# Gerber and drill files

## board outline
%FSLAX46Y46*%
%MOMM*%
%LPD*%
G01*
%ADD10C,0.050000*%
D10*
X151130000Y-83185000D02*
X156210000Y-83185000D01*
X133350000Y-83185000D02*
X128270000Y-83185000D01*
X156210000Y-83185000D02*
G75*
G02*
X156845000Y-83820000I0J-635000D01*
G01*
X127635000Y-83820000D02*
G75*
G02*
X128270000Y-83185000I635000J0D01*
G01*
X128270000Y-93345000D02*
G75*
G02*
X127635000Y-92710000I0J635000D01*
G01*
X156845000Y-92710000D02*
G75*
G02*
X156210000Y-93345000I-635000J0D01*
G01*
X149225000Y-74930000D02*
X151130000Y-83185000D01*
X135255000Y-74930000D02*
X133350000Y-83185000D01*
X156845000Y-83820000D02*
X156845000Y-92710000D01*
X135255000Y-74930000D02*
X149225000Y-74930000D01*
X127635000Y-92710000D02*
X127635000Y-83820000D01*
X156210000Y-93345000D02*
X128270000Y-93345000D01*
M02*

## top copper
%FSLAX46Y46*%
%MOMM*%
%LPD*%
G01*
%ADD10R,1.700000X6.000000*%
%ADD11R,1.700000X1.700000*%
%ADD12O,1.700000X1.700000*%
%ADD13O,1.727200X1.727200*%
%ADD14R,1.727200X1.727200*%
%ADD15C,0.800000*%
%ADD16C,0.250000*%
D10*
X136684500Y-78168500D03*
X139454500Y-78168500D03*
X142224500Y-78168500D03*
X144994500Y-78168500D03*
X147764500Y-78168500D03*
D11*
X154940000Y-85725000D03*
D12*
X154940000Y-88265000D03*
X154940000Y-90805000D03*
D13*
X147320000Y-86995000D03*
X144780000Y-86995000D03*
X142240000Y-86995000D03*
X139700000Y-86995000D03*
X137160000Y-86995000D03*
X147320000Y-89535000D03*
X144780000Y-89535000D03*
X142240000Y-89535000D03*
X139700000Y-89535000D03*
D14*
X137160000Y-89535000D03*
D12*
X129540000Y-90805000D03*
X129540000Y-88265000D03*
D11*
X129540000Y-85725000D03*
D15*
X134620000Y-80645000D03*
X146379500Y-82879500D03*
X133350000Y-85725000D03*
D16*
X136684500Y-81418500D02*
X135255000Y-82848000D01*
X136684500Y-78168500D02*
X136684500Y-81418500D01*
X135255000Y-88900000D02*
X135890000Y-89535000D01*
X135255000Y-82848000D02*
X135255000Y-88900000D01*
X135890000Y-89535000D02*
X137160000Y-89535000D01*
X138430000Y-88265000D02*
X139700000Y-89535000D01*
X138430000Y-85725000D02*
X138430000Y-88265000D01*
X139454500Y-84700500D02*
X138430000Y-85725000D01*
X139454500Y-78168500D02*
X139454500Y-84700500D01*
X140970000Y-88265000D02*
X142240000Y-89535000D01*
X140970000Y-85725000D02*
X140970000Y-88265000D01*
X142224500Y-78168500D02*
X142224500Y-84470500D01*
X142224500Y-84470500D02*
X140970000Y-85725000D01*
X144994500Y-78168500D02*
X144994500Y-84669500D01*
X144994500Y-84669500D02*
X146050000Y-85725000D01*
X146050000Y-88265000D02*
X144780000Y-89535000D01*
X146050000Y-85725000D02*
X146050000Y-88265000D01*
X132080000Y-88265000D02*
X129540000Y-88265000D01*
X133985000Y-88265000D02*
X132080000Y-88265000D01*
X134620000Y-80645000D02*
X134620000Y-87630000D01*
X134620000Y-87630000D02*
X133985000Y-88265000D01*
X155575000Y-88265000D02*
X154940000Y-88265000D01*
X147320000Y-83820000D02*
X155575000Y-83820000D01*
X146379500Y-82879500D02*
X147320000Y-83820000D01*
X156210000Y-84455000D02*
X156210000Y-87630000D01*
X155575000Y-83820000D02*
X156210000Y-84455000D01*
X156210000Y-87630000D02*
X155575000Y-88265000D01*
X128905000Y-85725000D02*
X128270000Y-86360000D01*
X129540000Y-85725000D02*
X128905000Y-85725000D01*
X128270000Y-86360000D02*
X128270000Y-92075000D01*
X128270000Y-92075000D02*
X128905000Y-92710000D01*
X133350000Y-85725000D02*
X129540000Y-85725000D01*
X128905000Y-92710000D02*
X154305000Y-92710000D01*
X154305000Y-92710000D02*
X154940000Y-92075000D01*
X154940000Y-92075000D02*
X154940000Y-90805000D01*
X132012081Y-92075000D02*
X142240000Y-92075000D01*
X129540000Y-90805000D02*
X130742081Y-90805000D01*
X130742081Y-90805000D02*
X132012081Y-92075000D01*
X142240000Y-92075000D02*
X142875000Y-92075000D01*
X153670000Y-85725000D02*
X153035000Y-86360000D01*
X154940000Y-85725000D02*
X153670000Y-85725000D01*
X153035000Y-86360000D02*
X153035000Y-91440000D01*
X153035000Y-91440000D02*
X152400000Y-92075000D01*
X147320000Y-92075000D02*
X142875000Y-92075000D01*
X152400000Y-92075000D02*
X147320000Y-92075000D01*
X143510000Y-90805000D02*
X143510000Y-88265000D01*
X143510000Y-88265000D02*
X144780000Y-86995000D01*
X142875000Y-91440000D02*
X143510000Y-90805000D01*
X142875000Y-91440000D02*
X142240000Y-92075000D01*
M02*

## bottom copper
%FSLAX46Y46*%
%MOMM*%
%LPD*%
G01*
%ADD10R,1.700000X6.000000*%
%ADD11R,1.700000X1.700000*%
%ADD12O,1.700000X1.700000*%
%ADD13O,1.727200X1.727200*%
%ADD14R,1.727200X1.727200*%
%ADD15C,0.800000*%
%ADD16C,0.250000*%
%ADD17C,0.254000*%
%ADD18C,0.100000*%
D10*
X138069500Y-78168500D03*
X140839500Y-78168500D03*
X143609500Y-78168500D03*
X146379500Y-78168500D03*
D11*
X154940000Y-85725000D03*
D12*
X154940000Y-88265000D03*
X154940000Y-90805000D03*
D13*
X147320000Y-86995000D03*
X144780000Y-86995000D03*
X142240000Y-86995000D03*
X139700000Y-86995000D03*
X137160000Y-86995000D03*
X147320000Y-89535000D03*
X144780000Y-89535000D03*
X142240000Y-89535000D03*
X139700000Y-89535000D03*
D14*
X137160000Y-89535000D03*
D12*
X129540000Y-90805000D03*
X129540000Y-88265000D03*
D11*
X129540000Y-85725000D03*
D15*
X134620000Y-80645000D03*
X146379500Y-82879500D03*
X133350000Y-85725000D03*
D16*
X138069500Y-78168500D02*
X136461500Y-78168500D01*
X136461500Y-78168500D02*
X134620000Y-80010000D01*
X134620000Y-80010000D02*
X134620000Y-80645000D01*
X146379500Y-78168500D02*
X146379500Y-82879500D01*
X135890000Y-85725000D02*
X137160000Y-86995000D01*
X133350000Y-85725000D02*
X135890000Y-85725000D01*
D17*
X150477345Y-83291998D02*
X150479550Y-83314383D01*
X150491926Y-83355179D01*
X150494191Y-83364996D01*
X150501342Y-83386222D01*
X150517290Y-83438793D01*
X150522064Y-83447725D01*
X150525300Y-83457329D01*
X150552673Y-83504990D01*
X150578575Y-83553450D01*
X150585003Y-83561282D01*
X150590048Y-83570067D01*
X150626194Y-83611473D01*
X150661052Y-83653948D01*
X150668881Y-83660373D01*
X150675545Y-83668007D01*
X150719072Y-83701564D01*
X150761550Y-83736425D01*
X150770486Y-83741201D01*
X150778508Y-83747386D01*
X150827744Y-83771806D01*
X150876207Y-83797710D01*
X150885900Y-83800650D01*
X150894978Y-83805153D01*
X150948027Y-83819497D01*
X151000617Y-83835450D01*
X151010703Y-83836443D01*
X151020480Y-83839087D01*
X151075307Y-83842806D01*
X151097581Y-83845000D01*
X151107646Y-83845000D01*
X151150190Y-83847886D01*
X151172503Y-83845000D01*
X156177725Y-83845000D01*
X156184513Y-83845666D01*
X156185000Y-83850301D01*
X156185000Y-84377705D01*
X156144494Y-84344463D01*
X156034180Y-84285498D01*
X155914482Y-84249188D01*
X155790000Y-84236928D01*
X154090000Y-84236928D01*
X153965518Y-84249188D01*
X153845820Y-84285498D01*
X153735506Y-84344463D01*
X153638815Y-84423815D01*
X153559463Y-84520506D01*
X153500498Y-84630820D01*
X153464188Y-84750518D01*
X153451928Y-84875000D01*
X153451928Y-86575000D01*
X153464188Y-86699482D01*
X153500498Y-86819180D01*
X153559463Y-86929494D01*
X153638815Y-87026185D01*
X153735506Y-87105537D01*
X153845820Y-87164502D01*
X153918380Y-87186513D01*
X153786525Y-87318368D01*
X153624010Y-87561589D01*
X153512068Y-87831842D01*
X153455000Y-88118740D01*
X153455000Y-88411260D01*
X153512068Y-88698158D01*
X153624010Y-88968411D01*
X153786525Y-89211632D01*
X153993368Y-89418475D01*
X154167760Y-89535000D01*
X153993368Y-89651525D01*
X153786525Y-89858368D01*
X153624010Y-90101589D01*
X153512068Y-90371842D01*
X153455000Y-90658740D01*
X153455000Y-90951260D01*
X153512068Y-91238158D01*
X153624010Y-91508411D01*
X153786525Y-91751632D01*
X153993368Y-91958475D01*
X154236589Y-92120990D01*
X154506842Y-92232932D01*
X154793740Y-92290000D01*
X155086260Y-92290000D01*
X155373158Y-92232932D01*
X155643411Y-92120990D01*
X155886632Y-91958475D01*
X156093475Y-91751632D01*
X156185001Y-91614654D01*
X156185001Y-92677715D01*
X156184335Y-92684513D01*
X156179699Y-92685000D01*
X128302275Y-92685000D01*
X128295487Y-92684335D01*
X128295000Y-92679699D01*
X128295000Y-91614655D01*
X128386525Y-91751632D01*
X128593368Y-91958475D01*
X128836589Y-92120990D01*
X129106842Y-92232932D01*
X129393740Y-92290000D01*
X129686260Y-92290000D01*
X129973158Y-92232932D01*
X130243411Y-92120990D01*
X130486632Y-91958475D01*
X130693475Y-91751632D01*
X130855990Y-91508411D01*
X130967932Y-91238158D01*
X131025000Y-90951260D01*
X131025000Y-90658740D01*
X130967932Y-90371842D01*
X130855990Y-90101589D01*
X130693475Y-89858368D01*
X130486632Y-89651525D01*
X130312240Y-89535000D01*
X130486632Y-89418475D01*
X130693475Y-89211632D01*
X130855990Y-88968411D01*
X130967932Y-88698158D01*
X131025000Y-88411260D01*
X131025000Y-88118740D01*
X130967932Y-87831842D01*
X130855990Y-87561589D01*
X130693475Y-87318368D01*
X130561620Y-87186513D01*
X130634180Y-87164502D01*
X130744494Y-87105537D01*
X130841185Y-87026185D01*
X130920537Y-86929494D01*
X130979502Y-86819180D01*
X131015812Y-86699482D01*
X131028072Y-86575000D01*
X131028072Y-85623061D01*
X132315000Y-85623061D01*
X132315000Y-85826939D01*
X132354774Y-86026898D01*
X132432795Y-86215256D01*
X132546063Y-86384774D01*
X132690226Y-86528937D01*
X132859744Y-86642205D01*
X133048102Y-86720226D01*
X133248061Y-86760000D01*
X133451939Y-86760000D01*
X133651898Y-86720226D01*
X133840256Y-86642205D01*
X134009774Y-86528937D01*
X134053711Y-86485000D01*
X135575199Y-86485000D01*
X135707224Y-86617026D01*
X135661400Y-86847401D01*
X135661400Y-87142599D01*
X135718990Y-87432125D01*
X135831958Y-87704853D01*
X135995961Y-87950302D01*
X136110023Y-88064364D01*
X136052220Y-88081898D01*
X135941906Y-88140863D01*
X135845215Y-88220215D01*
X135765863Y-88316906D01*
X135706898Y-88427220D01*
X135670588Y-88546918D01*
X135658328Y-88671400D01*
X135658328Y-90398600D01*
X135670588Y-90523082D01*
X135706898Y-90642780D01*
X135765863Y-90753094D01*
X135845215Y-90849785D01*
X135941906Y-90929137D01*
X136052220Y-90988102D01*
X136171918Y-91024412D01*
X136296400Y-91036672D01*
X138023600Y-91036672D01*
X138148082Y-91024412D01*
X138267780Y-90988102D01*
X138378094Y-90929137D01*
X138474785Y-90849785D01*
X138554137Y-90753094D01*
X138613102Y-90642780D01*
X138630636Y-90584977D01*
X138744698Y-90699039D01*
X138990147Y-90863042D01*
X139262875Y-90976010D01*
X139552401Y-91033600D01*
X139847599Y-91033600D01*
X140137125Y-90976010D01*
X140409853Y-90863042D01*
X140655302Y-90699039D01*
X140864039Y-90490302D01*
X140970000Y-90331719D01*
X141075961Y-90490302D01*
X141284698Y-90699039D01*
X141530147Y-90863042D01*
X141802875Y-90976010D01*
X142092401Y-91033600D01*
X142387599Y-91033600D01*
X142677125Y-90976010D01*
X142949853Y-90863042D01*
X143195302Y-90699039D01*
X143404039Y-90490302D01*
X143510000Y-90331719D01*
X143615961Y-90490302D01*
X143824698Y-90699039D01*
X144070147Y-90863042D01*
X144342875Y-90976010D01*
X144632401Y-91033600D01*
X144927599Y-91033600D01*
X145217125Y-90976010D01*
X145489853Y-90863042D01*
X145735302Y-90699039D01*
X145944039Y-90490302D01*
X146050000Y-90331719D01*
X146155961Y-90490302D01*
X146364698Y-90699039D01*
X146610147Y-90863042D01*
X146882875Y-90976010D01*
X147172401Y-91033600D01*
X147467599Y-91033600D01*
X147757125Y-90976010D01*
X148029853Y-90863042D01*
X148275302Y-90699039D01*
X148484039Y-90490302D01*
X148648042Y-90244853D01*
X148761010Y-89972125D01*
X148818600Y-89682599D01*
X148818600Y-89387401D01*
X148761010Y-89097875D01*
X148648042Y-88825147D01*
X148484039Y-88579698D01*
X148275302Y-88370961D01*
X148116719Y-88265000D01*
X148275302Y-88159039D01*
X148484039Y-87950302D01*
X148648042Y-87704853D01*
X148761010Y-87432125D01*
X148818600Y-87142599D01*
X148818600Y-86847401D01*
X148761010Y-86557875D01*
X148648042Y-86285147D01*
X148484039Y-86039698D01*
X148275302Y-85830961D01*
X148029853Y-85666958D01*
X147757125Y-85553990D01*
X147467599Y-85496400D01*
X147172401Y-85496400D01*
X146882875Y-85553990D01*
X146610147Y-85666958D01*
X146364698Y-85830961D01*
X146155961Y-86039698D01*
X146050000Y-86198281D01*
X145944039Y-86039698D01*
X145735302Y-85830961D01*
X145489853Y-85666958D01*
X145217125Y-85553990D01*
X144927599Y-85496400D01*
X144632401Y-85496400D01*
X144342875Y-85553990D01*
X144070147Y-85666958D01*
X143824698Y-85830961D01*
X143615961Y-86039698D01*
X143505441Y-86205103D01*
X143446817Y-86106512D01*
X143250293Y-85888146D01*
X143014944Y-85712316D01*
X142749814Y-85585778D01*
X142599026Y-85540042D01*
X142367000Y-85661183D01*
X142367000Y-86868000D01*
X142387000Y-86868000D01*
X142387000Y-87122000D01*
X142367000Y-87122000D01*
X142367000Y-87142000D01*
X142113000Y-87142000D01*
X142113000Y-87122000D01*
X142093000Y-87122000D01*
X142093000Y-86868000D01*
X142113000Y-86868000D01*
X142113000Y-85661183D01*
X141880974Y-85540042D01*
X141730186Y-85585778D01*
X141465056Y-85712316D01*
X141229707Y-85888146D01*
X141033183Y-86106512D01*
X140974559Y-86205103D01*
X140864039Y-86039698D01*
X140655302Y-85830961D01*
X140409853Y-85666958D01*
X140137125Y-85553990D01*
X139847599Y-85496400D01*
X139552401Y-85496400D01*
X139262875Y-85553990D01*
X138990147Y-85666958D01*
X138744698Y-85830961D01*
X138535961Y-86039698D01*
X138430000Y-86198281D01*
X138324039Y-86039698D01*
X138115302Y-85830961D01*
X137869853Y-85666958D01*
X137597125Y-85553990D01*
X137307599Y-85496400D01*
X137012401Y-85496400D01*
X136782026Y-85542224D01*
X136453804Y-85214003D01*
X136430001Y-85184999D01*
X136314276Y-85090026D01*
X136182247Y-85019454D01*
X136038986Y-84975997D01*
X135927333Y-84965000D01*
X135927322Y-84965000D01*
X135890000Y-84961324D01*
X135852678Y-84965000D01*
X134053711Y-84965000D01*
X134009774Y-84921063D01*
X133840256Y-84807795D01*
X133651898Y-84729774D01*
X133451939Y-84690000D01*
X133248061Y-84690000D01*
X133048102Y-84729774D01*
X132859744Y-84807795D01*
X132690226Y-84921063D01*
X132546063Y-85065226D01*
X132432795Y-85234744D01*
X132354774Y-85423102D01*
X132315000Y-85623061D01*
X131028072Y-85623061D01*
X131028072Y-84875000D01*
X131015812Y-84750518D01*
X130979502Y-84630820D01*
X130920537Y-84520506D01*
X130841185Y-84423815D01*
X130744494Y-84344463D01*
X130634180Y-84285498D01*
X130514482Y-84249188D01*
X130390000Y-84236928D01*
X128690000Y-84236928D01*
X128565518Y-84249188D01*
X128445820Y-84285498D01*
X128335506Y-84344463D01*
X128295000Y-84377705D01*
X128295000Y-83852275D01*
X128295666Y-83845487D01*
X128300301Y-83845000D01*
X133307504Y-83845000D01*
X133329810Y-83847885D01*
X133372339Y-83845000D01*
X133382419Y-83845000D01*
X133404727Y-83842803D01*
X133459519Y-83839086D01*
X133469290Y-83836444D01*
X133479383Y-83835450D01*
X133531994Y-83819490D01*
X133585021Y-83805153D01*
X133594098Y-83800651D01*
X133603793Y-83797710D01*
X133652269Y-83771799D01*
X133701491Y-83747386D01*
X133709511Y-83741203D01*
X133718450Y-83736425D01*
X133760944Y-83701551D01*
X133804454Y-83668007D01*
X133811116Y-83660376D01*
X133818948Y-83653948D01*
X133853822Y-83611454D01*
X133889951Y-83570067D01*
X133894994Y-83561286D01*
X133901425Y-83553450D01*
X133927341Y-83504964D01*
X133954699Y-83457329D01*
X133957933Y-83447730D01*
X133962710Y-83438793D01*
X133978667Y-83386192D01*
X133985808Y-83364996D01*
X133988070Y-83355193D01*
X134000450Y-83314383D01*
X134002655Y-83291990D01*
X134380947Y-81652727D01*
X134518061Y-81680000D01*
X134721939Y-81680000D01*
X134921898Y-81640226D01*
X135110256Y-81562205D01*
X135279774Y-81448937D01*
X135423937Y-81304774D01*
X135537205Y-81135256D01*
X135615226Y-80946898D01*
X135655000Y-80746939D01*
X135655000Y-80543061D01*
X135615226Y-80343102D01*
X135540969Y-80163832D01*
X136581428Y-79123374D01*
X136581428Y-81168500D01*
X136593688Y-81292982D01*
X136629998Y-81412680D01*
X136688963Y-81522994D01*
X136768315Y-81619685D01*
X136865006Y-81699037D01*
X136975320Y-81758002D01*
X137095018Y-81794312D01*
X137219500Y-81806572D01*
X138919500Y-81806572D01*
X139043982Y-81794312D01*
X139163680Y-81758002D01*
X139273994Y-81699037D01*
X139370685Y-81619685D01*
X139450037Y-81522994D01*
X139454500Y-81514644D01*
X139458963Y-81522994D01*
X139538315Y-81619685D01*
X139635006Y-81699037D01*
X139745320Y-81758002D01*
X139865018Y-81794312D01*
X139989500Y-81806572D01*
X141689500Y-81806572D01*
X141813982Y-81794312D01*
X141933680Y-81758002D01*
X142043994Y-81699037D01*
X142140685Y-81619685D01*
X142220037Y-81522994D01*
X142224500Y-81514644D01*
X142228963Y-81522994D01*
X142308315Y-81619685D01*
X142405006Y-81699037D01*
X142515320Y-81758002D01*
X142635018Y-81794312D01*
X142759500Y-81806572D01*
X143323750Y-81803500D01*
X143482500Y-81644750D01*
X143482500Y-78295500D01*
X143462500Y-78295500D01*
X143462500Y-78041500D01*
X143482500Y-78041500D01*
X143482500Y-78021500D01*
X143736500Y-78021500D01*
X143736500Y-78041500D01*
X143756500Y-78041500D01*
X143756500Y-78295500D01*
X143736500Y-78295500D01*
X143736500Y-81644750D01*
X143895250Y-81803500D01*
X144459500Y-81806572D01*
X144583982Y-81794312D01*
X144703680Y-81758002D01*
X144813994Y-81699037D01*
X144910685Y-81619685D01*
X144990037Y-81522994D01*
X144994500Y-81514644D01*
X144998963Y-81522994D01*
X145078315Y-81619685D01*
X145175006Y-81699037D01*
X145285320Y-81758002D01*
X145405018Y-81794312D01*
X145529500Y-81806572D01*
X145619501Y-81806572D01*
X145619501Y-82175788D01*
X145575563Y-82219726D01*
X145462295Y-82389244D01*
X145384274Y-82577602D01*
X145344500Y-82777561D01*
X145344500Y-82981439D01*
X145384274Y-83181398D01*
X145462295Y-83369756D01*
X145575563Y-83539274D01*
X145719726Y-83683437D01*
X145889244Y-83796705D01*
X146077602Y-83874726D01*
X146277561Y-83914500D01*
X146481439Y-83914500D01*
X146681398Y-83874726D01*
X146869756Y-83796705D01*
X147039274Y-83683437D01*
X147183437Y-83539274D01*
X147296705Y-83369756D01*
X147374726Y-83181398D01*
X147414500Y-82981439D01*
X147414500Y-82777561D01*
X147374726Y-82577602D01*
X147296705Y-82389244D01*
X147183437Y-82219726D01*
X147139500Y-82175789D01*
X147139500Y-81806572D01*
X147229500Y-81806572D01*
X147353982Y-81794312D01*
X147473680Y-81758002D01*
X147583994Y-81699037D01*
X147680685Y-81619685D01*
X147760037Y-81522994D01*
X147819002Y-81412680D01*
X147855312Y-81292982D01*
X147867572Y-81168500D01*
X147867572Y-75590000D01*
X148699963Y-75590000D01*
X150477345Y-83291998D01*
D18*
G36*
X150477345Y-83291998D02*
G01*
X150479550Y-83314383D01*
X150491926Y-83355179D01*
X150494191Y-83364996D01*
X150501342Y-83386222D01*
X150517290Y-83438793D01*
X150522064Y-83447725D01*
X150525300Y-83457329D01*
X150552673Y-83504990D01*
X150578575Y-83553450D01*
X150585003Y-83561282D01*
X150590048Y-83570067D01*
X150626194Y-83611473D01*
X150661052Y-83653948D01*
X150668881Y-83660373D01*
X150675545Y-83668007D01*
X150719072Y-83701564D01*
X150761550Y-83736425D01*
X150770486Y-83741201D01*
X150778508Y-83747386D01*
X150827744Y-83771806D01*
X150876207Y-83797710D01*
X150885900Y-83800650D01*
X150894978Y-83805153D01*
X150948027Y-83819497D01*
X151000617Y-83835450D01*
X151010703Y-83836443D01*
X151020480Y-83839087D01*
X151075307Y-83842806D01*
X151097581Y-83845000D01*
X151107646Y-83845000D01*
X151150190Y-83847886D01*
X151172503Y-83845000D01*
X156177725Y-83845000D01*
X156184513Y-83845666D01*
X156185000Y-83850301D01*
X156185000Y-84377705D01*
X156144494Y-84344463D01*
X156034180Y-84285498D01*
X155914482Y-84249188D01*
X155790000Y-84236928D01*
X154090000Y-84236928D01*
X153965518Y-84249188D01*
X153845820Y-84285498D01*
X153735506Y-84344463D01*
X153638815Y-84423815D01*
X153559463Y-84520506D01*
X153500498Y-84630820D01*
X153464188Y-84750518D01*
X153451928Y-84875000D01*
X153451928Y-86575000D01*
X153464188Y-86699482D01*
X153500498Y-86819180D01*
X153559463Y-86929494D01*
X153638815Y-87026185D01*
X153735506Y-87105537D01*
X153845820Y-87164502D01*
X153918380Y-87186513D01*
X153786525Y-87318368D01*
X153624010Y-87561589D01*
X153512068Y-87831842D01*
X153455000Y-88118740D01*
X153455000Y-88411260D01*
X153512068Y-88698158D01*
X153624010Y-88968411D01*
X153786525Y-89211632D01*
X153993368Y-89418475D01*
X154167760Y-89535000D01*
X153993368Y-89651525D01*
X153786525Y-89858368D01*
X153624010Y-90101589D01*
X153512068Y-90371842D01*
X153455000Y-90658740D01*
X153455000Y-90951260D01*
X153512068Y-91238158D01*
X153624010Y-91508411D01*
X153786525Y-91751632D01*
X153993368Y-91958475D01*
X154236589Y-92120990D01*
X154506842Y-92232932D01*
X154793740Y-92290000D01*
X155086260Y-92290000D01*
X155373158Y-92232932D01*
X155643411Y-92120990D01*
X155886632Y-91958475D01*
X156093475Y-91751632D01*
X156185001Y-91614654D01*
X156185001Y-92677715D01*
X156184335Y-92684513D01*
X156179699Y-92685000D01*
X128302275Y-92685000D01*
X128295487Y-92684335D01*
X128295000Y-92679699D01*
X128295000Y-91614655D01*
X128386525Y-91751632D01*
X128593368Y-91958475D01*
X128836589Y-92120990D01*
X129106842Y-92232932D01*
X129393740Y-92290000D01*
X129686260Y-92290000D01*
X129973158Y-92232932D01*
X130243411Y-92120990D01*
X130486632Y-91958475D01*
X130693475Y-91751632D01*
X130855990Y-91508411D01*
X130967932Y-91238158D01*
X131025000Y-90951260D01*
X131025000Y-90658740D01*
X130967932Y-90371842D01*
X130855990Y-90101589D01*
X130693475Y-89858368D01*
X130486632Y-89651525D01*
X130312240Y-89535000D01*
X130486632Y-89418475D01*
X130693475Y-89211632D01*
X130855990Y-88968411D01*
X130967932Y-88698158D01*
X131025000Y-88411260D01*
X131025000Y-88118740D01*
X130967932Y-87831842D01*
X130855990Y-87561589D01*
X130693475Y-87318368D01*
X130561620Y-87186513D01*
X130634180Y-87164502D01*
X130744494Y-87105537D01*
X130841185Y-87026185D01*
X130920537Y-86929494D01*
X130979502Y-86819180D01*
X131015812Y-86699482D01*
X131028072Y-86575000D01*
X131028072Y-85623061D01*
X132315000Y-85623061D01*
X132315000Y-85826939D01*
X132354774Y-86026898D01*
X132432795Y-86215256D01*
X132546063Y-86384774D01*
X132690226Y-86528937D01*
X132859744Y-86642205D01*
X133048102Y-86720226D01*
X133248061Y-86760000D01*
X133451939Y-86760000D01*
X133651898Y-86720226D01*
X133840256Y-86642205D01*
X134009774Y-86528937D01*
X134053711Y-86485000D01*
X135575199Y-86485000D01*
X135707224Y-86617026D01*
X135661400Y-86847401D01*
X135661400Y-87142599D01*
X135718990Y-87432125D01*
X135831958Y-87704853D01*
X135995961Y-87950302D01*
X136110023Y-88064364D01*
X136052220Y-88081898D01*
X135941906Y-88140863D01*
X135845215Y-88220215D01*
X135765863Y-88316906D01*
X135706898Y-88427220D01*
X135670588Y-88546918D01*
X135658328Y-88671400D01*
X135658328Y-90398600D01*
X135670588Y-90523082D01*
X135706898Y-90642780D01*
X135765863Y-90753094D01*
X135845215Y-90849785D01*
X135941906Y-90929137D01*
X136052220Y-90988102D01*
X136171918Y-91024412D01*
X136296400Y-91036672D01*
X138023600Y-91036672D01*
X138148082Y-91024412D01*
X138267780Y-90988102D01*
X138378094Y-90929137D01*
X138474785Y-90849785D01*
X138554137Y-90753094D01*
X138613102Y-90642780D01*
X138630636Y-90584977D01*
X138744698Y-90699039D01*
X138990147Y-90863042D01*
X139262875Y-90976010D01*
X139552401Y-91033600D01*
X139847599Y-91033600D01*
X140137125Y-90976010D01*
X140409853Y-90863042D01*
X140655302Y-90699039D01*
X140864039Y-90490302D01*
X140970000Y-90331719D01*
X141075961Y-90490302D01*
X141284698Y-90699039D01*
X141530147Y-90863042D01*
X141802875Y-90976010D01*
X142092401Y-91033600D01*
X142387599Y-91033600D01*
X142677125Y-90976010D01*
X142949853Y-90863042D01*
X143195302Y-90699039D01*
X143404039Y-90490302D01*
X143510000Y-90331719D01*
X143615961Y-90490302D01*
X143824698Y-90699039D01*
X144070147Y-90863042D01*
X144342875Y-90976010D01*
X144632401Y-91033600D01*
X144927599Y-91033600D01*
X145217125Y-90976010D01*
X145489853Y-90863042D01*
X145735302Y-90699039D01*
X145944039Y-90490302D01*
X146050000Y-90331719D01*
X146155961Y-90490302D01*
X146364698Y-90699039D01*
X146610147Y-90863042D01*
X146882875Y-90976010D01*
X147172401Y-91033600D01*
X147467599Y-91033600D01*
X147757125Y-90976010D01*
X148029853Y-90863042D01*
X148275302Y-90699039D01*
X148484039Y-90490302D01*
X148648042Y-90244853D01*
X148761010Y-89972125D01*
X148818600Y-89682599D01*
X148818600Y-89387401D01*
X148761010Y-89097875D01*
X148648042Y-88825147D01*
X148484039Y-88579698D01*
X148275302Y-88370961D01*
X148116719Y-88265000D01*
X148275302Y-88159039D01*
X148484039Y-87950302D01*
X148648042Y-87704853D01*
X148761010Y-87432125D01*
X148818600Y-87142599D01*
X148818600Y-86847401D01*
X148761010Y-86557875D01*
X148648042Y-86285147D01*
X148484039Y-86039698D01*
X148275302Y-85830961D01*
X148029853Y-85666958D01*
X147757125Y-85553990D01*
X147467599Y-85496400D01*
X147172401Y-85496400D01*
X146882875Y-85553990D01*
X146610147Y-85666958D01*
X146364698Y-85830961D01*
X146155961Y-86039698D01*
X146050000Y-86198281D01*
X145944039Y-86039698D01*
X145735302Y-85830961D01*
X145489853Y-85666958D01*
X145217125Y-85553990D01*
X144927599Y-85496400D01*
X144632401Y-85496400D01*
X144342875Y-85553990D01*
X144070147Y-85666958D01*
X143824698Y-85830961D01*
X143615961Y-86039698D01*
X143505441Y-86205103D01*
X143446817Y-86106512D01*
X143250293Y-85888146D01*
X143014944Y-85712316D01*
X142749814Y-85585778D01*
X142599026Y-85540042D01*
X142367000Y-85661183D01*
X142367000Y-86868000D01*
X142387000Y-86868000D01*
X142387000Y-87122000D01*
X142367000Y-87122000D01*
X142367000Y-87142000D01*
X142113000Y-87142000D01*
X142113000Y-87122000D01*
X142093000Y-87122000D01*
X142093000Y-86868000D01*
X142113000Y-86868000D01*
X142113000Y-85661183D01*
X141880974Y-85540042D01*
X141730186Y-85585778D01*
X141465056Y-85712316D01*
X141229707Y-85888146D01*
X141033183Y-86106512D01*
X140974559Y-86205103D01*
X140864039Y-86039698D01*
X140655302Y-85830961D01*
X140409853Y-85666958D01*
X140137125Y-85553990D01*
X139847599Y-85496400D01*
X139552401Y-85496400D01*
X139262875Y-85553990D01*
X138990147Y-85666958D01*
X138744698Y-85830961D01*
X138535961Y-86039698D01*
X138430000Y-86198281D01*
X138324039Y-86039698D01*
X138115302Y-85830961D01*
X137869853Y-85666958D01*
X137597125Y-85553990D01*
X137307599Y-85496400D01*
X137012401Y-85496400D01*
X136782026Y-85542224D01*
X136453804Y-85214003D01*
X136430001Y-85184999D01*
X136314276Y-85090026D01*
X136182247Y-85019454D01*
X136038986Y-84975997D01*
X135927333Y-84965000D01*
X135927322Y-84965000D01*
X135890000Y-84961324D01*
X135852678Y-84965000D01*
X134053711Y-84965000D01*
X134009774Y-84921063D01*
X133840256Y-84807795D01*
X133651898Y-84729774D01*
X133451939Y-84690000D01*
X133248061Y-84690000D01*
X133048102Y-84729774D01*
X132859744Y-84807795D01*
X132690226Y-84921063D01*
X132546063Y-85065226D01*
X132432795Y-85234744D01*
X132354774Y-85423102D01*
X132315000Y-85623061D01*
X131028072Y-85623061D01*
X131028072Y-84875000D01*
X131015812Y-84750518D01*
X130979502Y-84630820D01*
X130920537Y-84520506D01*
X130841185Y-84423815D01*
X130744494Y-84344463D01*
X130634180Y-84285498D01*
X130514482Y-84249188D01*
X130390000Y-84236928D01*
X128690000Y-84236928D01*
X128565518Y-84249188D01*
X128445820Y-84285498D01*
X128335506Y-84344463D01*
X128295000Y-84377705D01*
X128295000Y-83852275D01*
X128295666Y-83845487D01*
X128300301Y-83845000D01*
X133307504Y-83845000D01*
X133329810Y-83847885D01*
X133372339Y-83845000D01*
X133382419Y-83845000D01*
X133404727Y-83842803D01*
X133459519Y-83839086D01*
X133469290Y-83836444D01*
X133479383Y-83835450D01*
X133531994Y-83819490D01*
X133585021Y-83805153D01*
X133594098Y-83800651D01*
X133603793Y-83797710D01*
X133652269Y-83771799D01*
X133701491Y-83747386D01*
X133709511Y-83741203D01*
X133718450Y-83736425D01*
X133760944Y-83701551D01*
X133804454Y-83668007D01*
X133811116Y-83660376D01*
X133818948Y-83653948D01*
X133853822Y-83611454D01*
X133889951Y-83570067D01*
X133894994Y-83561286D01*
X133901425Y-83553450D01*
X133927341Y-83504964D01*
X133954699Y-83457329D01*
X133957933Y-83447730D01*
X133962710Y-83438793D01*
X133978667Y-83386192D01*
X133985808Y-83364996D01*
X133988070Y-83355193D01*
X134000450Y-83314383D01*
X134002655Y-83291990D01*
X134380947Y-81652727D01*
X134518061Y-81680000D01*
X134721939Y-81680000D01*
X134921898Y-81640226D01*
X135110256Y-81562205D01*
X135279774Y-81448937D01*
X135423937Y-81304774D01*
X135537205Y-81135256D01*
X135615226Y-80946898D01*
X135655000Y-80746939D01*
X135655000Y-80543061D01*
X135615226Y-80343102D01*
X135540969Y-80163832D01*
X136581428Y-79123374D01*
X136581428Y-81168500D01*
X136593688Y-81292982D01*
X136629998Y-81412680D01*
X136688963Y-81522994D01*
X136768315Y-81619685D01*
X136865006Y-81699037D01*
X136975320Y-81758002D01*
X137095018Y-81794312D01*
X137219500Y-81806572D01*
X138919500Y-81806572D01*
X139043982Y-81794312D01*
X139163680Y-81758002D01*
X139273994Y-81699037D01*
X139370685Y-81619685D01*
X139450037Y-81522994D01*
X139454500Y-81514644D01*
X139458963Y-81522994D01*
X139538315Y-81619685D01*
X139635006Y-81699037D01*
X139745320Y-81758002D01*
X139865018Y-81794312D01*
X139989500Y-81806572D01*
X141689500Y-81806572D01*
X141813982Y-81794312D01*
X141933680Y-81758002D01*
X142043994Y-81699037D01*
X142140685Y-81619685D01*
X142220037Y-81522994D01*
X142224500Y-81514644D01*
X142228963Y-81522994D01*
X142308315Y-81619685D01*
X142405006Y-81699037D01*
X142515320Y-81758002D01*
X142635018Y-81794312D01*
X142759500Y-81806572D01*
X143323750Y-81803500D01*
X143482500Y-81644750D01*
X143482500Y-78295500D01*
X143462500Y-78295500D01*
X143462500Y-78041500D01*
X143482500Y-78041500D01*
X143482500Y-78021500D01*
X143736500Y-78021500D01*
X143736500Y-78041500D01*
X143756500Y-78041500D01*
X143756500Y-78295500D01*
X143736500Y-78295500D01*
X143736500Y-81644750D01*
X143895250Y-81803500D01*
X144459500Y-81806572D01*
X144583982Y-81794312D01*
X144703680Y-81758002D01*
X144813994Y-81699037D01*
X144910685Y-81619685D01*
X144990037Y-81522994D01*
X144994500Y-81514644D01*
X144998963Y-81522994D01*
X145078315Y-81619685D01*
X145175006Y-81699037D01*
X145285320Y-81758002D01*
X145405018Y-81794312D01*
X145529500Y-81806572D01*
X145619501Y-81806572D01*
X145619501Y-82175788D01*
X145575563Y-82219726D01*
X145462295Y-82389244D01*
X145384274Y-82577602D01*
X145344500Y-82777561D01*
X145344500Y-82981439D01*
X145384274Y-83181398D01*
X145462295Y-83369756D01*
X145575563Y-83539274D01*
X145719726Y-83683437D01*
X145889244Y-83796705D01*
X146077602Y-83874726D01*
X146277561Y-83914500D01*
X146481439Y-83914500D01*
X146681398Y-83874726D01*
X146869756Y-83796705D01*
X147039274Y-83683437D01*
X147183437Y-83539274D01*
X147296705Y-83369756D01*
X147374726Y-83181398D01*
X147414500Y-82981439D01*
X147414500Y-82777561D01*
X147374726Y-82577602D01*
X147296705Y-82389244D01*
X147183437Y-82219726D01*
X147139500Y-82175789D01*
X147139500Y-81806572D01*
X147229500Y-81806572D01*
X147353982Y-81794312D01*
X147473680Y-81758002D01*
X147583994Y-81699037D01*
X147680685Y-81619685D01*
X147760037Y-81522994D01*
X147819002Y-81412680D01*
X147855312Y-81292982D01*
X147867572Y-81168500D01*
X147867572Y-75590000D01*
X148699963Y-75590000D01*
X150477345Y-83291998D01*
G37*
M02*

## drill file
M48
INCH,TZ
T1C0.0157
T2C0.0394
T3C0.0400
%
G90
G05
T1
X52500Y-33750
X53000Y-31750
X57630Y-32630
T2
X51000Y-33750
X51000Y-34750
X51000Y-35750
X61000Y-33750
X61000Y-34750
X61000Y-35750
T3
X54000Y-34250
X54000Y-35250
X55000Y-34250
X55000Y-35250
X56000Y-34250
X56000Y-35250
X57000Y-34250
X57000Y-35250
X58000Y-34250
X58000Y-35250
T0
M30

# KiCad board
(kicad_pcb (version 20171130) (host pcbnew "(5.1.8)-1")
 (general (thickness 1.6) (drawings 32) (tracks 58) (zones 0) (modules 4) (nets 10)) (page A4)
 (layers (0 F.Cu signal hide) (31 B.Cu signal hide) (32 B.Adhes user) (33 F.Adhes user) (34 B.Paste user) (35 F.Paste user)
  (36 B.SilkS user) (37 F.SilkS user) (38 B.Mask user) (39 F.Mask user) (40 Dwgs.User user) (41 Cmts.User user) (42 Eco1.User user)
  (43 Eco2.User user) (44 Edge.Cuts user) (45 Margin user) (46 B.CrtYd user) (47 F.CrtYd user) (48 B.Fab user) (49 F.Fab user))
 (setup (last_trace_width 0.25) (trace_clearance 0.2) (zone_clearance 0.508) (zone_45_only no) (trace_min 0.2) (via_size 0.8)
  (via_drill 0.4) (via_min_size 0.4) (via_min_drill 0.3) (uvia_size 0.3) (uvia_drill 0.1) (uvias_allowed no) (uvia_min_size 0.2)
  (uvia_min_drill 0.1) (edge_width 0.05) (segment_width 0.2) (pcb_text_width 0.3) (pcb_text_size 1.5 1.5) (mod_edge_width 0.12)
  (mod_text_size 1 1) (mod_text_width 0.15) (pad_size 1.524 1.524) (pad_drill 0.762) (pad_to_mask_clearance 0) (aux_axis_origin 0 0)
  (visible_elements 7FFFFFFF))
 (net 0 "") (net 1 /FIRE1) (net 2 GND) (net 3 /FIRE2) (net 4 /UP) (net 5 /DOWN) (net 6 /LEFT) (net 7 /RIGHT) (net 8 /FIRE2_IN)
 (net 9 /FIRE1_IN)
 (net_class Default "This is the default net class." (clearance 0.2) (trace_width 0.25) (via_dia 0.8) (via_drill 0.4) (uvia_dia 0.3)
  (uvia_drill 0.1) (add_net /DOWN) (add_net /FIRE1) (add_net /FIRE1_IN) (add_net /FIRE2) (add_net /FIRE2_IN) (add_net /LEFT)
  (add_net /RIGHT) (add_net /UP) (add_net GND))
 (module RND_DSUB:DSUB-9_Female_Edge (layer F.Cu) (at 142.24 78.105)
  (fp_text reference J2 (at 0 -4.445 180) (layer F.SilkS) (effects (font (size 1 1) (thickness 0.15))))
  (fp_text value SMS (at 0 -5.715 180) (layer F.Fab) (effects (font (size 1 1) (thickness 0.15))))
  (pad 6 smd rect (at -4.1705 0.0635 180) (size 1.7 6) (layers B.Cu B.Paste B.Mask) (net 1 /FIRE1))
  (pad 7 smd rect (at -1.4005 0.0635 180) (size 1.7 6) (layers B.Cu B.Paste B.Mask))
  (pad 8 smd rect (at 1.3695 0.0635 180) (size 1.7 6) (layers B.Cu B.Paste B.Mask) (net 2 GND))
  (pad 9 smd rect (at 4.1395 0.0635 180) (size 1.7 6) (layers B.Cu B.Paste B.Mask) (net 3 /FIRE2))
  (pad 1 smd rect (at -5.5555 0.0635 180) (size 1.7 6) (layers F.Cu F.Paste F.Mask) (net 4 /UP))
  (pad 2 smd rect (at -2.7855 0.0635 180) (size 1.7 6) (layers F.Cu F.Paste F.Mask) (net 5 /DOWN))
  (pad 3 smd rect (at -0.0155 0.0635 180) (size 1.7 6) (layers F.Cu F.Paste F.Mask) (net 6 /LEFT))
  (pad 4 smd rect (at 2.7545 0.0635 180) (size 1.7 6) (layers F.Cu F.Paste F.Mask) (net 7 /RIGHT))
  (pad 5 smd rect (at 5.5245 0.0635 180) (size 1.7 6) (layers F.Cu F.Paste F.Mask)))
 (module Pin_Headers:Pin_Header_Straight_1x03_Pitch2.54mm (layer F.Cu) (at 154.94 85.725)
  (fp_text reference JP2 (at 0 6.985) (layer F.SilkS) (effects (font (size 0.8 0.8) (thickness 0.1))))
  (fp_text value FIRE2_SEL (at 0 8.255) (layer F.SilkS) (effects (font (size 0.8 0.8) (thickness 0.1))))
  (pad 1 thru_hole rect (at 0 0) (size 1.7 1.7) (drill 1) (layers *.Cu *.Mask) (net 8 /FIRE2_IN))
  (pad 2 thru_hole oval (at 0 2.54) (size 1.7 1.7) (drill 1) (layers *.Cu *.Mask) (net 3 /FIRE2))
  (pad 3 thru_hole oval (at 0 5.08) (size 1.7 1.7) (drill 1) (layers *.Cu *.Mask) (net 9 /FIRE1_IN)))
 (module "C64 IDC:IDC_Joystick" (layer F.Cu) (at 137.16 89.535 90)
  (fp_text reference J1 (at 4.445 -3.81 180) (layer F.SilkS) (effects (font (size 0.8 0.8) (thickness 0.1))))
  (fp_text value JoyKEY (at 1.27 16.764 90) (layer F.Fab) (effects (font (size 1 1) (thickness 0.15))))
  (pad 10 thru_hole oval (at 2.54 10.16 90) (size 1.7272 1.7272) (drill 1.016) (layers *.Cu *.Mask))
  (pad 9 thru_hole oval (at 2.54 7.62 90) (size 1.7272 1.7272) (drill 1.016) (layers *.Cu *.Mask) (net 8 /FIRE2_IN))
  (pad 8 thru_hole oval (at 2.54 5.08 90) (size 1.7272 1.7272) (drill 1.016) (layers *.Cu *.Mask) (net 2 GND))
  (pad 7 thru_hole oval (at 2.54 2.54 90) (size 1.7272 1.7272) (drill 1.016) (layers *.Cu *.Mask))
  (pad 6 thru_hole oval (at 2.54 0 90) (size 1.7272 1.7272) (drill 1.016) (layers *.Cu *.Mask) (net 9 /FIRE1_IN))
  (pad 5 thru_hole oval (at 0 10.16 90) (size 1.7272 1.7272) (drill 1.016) (layers *.Cu *.Mask))
  (pad 4 thru_hole oval (at 0 7.62 90) (size 1.7272 1.7272) (drill 1.016) (layers *.Cu *.Mask) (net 7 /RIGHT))
  (pad 3 thru_hole oval (at 0 5.08 90) (size 1.7272 1.7272) (drill 1.016) (layers *.Cu *.Mask) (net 6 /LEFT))
  (pad 2 thru_hole oval (at 0 2.54 90) (size 1.7272 1.7272) (drill 1.016) (layers *.Cu *.Mask) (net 5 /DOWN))
  (pad 1 thru_hole rect (at 0 0 90) (size 1.7272 1.7272) (drill 1.016) (layers *.Cu *.Mask) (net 4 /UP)))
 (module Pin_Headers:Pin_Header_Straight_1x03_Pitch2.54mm (layer F.Cu) (at 129.54 85.725)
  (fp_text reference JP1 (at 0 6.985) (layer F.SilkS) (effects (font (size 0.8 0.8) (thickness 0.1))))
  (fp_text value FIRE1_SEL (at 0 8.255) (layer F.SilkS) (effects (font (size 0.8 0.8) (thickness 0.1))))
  (pad 3 thru_hole oval (at 0 5.08) (size 1.7 1.7) (drill 1) (layers *.Cu *.Mask) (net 8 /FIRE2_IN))
  (pad 2 thru_hole oval (at 0 2.54) (size 1.7 1.7) (drill 1) (layers *.Cu *.Mask) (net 1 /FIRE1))
  (pad 1 thru_hole rect (at 0 0) (size 1.7 1.7) (drill 1) (layers *.Cu *.Mask) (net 9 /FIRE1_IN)))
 (gr_line (start 151.13 83.185) (end 156.21 83.185) (layer Edge.Cuts) (width 0.05))
 (gr_line (start 133.35 83.185) (end 128.27 83.185) (layer Edge.Cuts) (width 0.05))
 (gr_arc (start 156.21 83.82) (end 156.845 83.82) (angle -90) (layer Edge.Cuts) (width 0.05))
 (gr_arc (start 128.27 83.82) (end 128.27 83.185) (angle -90) (layer Edge.Cuts) (width 0.05))
 (gr_arc (start 128.27 92.71) (end 127.635 92.71) (angle -90) (layer Edge.Cuts) (width 0.05))
 (gr_arc (start 156.21 92.71) (end 156.21 93.345) (angle -90) (layer Edge.Cuts) (width 0.05))
 (gr_line (start 149.225 74.93) (end 151.13 83.185) (layer Edge.Cuts) (width 0.05))
 (gr_line (start 135.255 74.93) (end 133.35 83.185) (layer Edge.Cuts) (width 0.05))
 (gr_line (start 156.845 83.82) (end 156.845 92.71) (layer Edge.Cuts) (width 0.05))
 (gr_line (start 135.255 74.93) (end 149.225 74.93) (layer Edge.Cuts) (width 0.05))
 (gr_line (start 127.635 92.71) (end 127.635 83.82) (layer Edge.Cuts) (width 0.05))
 (gr_line (start 156.21 93.345) (end 128.27 93.345) (layer Edge.Cuts) (width 0.05))
 (segment (start 136.6845 81.4185) (end 135.255 82.848) (width 0.25) (layer F.Cu) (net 4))
 (segment (start 136.6845 78.1685) (end 136.6845 81.4185) (width 0.25) (layer F.Cu) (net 4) (status 10))
 (segment (start 135.255 88.9) (end 135.89 89.535) (width 0.25) (layer F.Cu) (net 4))
 (segment (start 135.255 82.848) (end 135.255 88.9) (width 0.25) (layer F.Cu) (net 4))
 (segment (start 135.89 89.535) (end 137.16 89.535) (width 0.25) (layer F.Cu) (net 4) (status 20))
 (segment (start 138.43 88.265) (end 139.7 89.535) (width 0.25) (layer F.Cu) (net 5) (status 20))
 (segment (start 138.43 85.725) (end 138.43 88.265) (width 0.25) (layer F.Cu) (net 5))
 (segment (start 139.4545 84.7005) (end 138.43 85.725) (width 0.25) (layer F.Cu) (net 5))
 (segment (start 139.4545 78.1685) (end 139.4545 84.7005) (width 0.25) (layer F.Cu) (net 5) (status 10))
 (segment (start 140.97 88.265) (end 142.24 89.535) (width 0.25) (layer F.Cu) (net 6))
 (segment (start 140.97 85.725) (end 140.97 88.265) (width 0.25) (layer F.Cu) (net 6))
 (segment (start 142.2245 78.1685) (end 142.2245 84.4705) (width 0.25) (layer F.Cu) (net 6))
 (segment (start 142.2245 84.4705) (end 140.97 85.725) (width 0.25) (layer F.Cu) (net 6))
 (segment (start 144.9945 78.1685) (end 144.9945 84.6695) (width 0.25) (layer F.Cu) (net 7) (status 10))
 (segment (start 144.9945 84.6695) (end 146.05 85.725) (width 0.25) (layer F.Cu) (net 7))
 (segment (start 146.05 88.265) (end 144.78 89.535) (width 0.25) (layer F.Cu) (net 7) (status 20))
 (segment (start 146.05 85.725) (end 146.05 88.265) (width 0.25) (layer F.Cu) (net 7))
 (segment (start 138.0695 78.1685) (end 136.4615 78.1685) (width 0.25) (layer B.Cu) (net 1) (status 10))
 (via (at 134.62 80.645) (size 0.8) (drill 0.4) (layers F.Cu B.Cu) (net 1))
 (segment (start 136.4615 78.1685) (end 134.62 80.01) (width 0.25) (layer B.Cu) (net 1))
 (segment (start 134.62 80.01) (end 134.62 80.645) (width 0.25) (layer B.Cu) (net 1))
 (segment (start 132.08 88.265) (end 129.54 88.265) (width 0.25) (layer F.Cu) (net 1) (status 20))
 (segment (start 133.985 88.265) (end 132.08 88.265) (width 0.25) (layer F.Cu) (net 1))
 (segment (start 134.62 80.645) (end 134.62 87.63) (width 0.25) (layer F.Cu) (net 1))
 (segment (start 134.62 87.63) (end 133.985 88.265) (width 0.25) (layer F.Cu) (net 1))
 (segment (start 146.3795 78.1685) (end 146.3795 82.8795) (width 0.25) (layer B.Cu) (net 3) (status 10))
 (via (at 146.3795 82.8795) (size 0.8) (drill 0.4) (layers F.Cu B.Cu) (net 3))
 (segment (start 155.575 88.265) (end 154.94 88.265) (width 0.25) (layer F.Cu) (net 3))
 (segment (start 147.32 83.82) (end 155.575 83.82) (width 0.25) (layer F.Cu) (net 3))
 (segment (start 146.3795 82.8795) (end 147.32 83.82) (width 0.25) (layer F.Cu) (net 3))
 (segment (start 156.21 84.455) (end 156.21 87.63) (width 0.25) (layer F.Cu) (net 3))
 (segment (start 155.575 83.82) (end 156.21 84.455) (width 0.25) (layer F.Cu) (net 3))
 (segment (start 156.21 87.63) (end 155.575 88.265) (width 0.25) (layer F.Cu) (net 3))
 (segment (start 135.89 85.725) (end 137.16 86.995) (width 0.25) (layer B.Cu) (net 9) (status 20))
 (segment (start 128.905 85.725) (end 128.27 86.36) (width 0.25) (layer F.Cu) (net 9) (status 10))
 (segment (start 129.54 85.725) (end 128.905 85.725) (width 0.25) (layer F.Cu) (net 9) (status 30))
 (segment (start 128.27 86.36) (end 128.27 92.075) (width 0.25) (layer F.Cu) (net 9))
 (segment (start 128.27 92.075) (end 128.905 92.71) (width 0.25) (layer F.Cu) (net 9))
 (via (at 133.35 85.725) (size 0.8) (drill 0.4) (layers F.Cu B.Cu) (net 9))
 (segment (start 133.35 85.725) (end 135.89 85.725) (width 0.25) (layer B.Cu) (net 9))
 (segment (start 133.35 85.725) (end 129.54 85.725) (width 0.25) (layer F.Cu) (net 9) (status 20))
 (segment (start 128.905 92.71) (end 154.305 92.71) (width 0.25) (layer F.Cu) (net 9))
 (segment (start 154.305 92.71) (end 154.94 92.075) (width 0.25) (layer F.Cu) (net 9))
 (segment (start 154.94 92.075) (end 154.94 90.805) (width 0.25) (layer F.Cu) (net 9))
 (segment (start 132.012081 92.075) (end 142.24 92.075) (width 0.25) (layer F.Cu) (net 8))
 (segment (start 129.54 90.805) (end 130.742081 90.805) (width 0.25) (layer F.Cu) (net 8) (status 10))
 (segment (start 130.742081 90.805) (end 132.012081 92.075) (width 0.25) (layer F.Cu) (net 8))
 (segment (start 142.24 92.075) (end 142.875 92.075) (width 0.25) (layer F.Cu) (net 8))
 (segment (start 153.67 85.725) (end 153.035 86.36) (width 0.25) (layer F.Cu) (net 8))
 (segment (start 154.94 85.725) (end 153.67 85.725) (width 0.25) (layer F.Cu) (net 8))
 (segment (start 153.035 86.36) (end 153.035 91.44) (width 0.25) (layer F.Cu) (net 8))
 (segment (start 153.035 91.44) (end 152.4 92.075) (width 0.25) (layer F.Cu) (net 8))
 (segment (start 147.32 92.075) (end 142.875 92.075) (width 0.25) (layer F.Cu) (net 8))
 (segment (start 152.4 92.075) (end 147.32 92.075) (width 0.25) (layer F.Cu) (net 8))
 (segment (start 143.51 90.805) (end 143.51 88.265) (width 0.25) (layer F.Cu) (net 8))
 (segment (start 143.51 88.265) (end 144.78 86.995) (width 0.25) (layer F.Cu) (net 8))
 (segment (start 142.875 91.44) (end 143.51 90.805) (width 0.25) (layer F.Cu) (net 8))
 (segment (start 142.875 91.44) (end 142.24 92.075) (width 0.25) (layer F.Cu) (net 8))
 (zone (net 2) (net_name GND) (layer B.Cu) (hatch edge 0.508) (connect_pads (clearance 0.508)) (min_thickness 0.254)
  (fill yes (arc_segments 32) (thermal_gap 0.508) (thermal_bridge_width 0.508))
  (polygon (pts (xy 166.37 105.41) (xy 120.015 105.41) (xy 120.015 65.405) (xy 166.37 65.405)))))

